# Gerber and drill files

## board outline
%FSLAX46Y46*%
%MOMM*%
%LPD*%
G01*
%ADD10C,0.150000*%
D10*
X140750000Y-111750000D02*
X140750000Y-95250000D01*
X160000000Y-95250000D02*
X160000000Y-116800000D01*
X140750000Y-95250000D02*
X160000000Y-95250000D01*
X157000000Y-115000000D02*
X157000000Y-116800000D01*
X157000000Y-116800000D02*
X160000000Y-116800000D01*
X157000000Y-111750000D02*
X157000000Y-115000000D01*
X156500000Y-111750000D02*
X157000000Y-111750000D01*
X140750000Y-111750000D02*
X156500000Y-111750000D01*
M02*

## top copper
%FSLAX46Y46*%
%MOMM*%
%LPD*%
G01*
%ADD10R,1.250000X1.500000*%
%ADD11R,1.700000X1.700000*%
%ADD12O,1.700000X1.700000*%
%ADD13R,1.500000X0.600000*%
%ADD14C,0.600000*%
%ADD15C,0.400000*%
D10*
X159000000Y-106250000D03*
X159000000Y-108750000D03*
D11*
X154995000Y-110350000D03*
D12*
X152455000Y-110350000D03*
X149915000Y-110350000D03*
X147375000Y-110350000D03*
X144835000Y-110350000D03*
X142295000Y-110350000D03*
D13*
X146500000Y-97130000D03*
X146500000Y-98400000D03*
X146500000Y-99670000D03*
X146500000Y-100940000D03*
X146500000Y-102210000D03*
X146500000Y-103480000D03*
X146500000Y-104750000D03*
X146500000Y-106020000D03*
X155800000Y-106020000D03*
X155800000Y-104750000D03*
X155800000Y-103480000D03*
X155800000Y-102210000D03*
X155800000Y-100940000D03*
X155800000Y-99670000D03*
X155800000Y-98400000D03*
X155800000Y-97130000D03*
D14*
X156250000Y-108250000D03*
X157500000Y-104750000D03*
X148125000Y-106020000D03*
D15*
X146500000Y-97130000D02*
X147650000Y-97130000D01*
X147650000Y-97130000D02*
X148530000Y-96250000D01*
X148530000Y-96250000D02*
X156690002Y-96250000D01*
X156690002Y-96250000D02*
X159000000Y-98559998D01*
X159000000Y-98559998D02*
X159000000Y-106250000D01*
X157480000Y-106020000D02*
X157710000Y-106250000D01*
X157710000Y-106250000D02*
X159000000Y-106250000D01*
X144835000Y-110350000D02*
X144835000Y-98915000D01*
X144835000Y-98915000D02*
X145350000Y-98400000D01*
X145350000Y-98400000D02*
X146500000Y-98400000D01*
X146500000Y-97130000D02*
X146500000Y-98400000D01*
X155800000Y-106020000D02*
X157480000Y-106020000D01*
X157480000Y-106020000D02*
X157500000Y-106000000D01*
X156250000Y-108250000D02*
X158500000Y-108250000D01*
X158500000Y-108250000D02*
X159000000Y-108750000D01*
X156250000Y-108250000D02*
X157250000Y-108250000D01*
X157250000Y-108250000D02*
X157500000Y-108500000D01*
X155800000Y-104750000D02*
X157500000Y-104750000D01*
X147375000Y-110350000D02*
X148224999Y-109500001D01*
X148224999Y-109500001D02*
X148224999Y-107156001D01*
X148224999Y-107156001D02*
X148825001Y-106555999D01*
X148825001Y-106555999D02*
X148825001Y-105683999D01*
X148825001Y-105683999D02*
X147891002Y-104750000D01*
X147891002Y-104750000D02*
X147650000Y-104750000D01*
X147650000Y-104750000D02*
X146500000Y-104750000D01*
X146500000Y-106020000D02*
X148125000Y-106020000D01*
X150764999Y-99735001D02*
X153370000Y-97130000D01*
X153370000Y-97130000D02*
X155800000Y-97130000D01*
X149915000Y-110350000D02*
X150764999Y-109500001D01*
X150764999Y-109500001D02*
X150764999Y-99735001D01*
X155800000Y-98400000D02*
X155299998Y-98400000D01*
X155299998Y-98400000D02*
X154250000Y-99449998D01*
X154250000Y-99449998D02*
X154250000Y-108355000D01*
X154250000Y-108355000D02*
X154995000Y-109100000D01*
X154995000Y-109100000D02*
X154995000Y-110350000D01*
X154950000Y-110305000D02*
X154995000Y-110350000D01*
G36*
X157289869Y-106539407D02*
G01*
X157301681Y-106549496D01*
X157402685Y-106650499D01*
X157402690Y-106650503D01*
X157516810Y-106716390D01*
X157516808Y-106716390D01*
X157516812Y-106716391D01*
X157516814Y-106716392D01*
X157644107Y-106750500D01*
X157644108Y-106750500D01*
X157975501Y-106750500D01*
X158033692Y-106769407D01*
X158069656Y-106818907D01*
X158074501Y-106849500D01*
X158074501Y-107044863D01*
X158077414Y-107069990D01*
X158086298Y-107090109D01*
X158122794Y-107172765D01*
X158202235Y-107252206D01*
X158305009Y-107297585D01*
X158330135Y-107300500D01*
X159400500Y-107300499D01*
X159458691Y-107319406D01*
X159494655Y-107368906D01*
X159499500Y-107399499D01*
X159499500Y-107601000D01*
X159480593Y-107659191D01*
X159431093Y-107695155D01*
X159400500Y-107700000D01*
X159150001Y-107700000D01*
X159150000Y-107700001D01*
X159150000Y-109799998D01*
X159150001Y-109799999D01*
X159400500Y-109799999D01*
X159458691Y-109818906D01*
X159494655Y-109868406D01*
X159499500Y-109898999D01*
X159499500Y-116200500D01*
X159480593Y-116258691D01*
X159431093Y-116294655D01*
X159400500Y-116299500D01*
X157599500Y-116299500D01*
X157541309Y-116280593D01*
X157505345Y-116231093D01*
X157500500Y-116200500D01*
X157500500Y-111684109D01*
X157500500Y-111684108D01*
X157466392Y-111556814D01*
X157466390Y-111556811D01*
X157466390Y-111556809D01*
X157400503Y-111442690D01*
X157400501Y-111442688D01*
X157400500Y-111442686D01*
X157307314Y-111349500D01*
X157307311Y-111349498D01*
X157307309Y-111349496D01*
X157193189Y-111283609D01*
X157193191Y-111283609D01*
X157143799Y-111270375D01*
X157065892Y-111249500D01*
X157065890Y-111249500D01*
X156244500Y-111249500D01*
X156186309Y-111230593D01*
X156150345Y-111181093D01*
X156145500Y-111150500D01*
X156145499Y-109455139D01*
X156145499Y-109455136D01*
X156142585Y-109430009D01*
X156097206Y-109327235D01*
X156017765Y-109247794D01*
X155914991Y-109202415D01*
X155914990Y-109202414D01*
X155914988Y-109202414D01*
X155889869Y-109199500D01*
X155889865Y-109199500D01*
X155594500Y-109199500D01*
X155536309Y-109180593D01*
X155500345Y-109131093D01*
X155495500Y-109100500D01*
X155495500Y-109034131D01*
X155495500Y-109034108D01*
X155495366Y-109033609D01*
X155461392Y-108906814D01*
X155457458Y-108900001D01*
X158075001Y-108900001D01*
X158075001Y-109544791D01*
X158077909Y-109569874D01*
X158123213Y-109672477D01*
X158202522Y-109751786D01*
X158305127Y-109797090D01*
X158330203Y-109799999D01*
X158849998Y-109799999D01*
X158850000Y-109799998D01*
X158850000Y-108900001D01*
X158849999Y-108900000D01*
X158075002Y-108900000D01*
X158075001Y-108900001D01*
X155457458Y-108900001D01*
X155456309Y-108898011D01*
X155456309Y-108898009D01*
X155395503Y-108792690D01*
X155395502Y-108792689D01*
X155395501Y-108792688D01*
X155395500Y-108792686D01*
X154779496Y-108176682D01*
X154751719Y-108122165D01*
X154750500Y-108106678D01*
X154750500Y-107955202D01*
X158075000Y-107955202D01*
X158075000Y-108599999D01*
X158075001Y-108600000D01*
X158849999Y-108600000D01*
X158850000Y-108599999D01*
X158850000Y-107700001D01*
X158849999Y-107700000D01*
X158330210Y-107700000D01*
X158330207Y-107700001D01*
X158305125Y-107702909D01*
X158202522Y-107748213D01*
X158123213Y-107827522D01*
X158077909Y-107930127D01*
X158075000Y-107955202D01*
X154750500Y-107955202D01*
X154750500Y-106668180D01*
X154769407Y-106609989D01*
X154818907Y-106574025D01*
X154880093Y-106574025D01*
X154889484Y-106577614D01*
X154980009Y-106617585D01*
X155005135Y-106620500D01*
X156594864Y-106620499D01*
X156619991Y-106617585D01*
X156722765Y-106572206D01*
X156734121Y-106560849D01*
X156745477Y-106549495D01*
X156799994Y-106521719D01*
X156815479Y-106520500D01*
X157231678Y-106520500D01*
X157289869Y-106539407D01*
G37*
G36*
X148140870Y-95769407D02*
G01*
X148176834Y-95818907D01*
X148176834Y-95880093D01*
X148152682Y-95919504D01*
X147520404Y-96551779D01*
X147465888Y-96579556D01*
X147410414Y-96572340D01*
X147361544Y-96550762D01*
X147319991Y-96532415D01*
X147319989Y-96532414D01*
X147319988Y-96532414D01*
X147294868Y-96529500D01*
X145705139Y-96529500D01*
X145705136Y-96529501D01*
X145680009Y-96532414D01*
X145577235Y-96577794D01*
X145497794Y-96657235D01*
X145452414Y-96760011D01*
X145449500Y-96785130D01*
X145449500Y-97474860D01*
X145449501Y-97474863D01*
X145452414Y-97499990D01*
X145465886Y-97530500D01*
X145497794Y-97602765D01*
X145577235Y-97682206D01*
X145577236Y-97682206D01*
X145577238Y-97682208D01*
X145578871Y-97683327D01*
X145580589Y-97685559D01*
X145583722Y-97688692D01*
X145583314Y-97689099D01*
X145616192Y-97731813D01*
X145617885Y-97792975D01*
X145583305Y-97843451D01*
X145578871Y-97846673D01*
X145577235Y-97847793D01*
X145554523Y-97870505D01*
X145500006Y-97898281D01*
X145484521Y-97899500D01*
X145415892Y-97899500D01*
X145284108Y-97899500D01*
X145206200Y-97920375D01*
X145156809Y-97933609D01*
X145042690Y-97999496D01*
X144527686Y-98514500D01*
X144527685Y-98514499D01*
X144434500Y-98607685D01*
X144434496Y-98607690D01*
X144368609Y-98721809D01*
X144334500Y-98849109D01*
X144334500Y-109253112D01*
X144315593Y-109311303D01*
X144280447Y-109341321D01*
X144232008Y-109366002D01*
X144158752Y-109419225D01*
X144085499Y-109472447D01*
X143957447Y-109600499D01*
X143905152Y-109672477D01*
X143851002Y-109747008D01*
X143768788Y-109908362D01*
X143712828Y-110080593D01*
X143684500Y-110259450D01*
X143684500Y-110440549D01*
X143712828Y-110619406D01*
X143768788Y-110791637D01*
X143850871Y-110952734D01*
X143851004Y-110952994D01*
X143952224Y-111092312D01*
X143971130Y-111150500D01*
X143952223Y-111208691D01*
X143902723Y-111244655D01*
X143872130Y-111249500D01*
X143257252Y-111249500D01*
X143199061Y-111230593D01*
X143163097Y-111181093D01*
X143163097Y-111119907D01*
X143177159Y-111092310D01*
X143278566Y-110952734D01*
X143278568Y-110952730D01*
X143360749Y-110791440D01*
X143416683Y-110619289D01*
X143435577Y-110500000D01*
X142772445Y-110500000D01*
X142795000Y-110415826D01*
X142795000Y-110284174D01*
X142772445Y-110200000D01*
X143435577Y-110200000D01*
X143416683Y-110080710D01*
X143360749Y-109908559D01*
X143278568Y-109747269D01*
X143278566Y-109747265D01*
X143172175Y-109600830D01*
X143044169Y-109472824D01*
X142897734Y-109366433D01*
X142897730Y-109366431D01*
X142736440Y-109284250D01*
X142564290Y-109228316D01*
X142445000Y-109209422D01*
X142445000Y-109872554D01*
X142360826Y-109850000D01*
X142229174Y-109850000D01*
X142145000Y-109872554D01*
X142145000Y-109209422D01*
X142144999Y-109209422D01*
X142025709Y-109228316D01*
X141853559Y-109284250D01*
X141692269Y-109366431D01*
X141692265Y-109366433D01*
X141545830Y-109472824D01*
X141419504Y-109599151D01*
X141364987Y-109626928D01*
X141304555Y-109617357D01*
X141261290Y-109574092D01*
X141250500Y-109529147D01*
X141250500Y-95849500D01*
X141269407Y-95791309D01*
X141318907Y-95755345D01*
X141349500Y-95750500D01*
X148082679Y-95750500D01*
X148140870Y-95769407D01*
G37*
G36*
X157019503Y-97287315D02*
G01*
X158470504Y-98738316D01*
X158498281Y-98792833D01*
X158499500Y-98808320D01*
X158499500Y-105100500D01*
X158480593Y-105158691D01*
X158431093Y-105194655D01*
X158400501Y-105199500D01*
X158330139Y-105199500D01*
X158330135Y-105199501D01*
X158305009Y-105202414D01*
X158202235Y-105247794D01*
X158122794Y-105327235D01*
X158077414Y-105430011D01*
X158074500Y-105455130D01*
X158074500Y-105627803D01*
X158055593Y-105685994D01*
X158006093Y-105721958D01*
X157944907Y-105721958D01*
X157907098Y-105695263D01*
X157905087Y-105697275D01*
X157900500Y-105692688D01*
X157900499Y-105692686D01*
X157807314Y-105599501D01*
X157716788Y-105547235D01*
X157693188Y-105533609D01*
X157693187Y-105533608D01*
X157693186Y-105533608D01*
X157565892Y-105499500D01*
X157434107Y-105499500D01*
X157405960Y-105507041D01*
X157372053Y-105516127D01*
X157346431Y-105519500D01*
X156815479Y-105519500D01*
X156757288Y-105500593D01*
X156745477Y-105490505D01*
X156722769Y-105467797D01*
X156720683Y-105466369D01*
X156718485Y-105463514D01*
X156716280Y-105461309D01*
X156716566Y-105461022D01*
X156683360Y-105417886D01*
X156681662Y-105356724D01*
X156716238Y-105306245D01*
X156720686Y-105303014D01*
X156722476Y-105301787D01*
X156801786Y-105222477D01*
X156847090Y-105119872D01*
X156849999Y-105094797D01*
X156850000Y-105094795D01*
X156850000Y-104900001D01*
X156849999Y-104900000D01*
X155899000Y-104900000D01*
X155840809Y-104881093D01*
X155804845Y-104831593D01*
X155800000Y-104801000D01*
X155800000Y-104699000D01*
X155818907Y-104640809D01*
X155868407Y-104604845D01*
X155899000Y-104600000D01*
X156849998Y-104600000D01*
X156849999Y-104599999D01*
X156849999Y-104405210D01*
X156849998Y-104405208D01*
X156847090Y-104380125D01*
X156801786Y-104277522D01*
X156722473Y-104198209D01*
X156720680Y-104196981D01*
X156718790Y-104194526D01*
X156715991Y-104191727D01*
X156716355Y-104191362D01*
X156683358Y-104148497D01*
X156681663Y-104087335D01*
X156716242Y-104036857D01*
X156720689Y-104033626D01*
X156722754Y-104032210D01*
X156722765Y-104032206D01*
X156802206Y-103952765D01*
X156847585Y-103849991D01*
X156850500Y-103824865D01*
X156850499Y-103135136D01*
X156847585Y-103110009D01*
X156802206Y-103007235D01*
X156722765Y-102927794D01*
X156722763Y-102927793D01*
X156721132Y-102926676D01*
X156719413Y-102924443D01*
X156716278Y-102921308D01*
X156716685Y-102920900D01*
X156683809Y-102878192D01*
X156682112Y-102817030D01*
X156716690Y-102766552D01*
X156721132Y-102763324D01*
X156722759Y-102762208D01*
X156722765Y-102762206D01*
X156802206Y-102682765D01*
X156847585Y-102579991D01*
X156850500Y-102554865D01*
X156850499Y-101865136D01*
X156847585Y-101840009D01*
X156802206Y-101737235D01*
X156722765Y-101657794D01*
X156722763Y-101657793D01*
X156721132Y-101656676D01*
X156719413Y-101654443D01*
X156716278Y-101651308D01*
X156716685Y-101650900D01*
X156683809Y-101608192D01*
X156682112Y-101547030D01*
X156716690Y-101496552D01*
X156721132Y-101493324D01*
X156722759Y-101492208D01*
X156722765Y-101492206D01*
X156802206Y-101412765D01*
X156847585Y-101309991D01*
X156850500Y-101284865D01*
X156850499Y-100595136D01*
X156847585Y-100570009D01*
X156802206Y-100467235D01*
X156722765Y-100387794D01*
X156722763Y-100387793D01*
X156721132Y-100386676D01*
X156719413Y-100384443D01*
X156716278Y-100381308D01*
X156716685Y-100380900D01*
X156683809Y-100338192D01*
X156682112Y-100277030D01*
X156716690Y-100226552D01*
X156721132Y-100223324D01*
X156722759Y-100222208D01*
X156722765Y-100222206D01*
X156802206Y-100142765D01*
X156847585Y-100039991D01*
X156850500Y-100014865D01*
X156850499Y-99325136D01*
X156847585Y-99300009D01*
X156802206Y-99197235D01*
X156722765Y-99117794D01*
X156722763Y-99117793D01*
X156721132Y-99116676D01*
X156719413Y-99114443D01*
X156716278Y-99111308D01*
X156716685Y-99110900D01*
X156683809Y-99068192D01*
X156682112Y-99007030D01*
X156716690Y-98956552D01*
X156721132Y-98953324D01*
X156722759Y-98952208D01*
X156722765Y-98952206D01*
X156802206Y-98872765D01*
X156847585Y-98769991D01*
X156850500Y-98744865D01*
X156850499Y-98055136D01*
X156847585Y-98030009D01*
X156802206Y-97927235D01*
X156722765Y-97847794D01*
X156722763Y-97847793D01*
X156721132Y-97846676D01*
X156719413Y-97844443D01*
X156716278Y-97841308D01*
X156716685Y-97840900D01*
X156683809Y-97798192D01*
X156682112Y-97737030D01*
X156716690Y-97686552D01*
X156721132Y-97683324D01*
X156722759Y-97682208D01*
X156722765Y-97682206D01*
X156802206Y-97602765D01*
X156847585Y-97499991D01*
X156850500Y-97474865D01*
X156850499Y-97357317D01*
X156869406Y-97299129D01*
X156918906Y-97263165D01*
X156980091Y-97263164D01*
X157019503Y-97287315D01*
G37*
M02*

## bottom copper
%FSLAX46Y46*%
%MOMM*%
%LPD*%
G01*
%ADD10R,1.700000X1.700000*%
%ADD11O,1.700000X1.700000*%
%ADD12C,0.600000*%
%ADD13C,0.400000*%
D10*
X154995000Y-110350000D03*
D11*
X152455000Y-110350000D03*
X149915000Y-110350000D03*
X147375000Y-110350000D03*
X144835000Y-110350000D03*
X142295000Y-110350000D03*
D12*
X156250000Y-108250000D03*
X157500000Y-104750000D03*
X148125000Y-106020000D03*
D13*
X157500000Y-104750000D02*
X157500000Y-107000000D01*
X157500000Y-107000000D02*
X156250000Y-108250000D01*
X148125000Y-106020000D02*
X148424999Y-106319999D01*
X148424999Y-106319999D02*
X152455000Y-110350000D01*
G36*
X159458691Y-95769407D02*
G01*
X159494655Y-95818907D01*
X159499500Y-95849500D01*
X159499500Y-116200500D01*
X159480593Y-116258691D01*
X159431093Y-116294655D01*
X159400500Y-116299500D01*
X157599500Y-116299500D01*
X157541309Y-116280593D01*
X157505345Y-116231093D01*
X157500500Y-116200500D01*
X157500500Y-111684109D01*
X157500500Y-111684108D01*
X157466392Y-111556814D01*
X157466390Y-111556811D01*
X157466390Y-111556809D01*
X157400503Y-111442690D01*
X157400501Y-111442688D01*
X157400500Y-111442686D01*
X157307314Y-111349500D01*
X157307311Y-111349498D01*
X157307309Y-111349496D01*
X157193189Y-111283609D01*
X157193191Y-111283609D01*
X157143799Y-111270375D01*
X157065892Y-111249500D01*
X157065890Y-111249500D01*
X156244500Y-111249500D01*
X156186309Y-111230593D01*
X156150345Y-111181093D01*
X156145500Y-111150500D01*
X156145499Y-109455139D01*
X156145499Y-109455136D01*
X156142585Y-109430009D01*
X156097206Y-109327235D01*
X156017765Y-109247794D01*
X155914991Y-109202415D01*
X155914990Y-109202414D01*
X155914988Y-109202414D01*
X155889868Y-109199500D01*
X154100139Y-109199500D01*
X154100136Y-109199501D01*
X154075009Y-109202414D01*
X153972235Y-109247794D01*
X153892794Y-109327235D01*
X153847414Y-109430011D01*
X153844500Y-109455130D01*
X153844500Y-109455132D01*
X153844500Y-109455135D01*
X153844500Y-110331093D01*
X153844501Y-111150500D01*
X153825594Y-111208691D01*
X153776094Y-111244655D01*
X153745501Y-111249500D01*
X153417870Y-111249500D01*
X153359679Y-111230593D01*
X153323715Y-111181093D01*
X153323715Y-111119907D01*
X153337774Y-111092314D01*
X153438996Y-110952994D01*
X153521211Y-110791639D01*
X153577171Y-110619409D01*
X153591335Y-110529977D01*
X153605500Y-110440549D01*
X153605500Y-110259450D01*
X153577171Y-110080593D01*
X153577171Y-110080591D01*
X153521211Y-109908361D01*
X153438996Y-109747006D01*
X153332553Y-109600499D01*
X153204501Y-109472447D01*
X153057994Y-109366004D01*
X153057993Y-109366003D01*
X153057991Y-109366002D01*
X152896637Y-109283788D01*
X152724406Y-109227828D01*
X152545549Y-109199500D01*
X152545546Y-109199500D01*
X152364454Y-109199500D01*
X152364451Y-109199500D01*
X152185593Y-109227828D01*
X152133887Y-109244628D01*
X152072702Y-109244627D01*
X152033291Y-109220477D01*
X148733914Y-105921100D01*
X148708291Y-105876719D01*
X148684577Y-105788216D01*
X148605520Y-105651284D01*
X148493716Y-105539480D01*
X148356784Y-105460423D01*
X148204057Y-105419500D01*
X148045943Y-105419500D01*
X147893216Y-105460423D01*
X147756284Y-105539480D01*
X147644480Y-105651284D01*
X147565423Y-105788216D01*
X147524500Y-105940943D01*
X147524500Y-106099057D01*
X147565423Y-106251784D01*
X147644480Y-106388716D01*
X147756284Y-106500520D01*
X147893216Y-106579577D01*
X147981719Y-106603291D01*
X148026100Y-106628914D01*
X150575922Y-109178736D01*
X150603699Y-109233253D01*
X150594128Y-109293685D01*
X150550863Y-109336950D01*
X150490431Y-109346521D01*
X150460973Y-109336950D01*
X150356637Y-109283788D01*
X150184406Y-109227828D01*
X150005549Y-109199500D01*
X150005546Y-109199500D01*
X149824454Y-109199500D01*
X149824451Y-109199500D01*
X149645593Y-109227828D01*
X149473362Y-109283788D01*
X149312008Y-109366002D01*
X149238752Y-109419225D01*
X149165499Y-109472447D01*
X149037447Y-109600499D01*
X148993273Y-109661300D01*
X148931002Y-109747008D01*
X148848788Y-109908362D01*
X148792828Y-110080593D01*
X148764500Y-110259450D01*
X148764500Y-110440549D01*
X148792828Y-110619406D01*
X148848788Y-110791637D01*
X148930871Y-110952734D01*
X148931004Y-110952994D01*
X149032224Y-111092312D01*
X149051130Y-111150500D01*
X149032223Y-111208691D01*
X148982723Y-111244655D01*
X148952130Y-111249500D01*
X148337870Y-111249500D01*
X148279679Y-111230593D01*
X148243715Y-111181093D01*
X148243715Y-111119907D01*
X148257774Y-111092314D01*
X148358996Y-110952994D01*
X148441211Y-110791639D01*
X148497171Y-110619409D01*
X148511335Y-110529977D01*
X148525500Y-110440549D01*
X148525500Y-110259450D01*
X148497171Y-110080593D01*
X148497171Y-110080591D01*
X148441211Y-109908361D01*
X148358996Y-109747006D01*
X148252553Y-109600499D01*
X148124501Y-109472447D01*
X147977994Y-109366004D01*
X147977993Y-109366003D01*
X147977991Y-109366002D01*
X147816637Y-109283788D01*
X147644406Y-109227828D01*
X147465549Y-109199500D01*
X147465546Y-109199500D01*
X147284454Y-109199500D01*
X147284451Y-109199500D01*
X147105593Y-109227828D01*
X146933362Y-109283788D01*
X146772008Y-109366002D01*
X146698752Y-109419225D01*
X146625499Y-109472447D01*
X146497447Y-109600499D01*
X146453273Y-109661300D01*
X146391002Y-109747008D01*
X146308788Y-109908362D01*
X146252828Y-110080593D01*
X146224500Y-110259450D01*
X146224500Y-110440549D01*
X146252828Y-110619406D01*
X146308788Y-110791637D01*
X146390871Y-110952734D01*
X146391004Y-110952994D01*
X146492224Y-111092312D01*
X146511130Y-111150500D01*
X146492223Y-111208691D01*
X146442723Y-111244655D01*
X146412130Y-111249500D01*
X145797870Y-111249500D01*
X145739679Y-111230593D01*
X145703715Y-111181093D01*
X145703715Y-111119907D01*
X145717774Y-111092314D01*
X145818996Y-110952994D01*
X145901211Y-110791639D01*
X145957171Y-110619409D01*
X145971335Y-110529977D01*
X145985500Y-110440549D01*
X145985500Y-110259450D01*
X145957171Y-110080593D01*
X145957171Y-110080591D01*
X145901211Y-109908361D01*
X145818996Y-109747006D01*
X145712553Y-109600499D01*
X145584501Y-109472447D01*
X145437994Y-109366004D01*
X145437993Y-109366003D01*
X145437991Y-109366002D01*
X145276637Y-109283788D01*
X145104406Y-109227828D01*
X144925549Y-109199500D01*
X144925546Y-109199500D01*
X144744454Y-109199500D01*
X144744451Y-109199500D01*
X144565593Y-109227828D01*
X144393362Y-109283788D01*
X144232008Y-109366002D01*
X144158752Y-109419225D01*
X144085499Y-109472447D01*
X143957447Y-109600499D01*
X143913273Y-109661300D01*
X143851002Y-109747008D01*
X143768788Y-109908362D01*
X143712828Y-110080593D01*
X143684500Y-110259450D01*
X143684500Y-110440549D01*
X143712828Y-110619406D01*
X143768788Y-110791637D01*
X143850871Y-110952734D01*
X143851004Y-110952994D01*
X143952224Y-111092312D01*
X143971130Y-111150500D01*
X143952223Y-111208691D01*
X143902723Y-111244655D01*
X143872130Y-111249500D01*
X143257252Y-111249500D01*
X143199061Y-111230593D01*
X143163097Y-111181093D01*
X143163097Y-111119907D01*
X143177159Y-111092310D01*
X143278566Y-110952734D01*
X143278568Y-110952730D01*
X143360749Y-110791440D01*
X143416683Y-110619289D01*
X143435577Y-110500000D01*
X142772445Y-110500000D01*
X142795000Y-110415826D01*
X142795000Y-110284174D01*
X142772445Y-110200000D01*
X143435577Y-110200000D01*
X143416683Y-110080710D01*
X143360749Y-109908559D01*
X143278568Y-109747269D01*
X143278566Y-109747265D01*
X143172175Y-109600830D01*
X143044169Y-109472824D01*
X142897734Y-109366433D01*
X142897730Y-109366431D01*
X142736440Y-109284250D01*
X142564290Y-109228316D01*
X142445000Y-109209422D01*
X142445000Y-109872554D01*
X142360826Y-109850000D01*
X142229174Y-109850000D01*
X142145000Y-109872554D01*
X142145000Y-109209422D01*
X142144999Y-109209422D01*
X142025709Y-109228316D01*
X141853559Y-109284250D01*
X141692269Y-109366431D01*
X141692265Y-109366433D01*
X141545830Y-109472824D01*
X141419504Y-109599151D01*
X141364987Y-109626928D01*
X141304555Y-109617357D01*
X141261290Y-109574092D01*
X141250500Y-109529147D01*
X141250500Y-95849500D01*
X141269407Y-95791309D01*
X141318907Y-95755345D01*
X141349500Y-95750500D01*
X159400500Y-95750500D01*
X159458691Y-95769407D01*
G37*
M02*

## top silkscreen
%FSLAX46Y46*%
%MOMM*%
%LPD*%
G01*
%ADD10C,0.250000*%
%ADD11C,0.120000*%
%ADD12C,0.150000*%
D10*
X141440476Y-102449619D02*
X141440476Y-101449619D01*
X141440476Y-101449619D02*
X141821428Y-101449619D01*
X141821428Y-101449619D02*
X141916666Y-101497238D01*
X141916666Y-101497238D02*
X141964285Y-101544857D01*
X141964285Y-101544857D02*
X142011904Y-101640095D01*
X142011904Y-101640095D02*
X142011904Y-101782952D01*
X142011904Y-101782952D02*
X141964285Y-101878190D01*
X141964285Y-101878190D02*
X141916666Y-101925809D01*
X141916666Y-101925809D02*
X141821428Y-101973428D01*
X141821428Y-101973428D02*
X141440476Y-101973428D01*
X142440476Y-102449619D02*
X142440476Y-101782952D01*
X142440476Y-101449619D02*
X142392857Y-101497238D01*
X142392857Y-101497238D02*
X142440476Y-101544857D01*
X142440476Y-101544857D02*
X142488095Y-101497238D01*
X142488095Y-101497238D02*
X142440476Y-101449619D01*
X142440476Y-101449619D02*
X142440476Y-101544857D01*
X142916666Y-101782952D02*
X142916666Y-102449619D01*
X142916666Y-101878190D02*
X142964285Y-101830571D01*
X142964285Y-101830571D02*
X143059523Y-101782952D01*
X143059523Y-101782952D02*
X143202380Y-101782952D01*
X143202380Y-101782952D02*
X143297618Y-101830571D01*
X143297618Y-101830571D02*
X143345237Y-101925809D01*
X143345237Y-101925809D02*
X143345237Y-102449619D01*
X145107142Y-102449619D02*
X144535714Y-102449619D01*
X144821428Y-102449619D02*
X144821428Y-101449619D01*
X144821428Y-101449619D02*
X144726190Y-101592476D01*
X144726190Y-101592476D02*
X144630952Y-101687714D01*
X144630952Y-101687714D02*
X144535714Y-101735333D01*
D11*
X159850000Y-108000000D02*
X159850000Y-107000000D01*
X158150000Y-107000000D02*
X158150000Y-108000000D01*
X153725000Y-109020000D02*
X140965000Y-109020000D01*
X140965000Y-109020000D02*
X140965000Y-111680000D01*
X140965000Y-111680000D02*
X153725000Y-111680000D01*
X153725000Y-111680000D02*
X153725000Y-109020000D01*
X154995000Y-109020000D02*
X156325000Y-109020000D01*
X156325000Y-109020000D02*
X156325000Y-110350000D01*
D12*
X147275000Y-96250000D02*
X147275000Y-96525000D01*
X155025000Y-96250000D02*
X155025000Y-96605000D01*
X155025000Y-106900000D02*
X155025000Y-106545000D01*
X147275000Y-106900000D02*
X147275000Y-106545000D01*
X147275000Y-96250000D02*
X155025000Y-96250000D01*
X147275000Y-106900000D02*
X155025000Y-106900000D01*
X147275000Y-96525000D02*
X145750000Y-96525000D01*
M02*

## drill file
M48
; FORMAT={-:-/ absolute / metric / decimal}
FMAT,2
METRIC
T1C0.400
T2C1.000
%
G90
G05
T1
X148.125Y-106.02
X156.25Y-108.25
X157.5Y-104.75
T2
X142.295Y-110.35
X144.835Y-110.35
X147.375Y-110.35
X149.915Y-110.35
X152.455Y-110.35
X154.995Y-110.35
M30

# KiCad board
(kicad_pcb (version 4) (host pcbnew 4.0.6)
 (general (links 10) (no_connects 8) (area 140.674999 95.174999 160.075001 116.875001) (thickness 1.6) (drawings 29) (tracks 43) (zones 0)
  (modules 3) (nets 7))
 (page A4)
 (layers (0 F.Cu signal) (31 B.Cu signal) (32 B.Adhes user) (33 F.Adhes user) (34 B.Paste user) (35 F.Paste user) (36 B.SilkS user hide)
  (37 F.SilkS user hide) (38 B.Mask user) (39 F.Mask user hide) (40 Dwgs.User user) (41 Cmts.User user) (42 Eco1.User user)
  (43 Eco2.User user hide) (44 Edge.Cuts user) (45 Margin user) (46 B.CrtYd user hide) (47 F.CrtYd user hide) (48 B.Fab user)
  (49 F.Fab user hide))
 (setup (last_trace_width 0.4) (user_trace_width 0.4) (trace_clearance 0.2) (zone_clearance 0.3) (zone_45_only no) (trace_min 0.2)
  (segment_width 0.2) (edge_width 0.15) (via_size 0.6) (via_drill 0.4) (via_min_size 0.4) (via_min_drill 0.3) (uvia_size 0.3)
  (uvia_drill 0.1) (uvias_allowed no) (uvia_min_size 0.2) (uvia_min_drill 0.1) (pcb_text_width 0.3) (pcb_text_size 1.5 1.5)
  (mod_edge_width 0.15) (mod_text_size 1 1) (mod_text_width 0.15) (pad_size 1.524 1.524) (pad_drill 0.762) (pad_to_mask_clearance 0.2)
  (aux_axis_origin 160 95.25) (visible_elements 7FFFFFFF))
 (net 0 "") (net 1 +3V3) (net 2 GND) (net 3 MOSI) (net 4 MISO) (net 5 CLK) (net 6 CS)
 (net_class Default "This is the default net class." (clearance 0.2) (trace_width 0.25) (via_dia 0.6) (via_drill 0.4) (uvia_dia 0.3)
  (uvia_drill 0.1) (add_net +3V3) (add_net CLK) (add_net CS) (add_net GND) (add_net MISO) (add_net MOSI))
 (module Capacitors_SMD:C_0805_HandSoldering (layer F.Cu) (at 159 107.5 270)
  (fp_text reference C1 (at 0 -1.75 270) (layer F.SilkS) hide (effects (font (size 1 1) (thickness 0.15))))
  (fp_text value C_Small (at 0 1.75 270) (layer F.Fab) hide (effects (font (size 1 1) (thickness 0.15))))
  (fp_line (start 0.5 -0.85) (end -0.5 -0.85) (layer F.SilkS) (width 0.12))
  (fp_line (start -0.5 0.85) (end 0.5 0.85) (layer F.SilkS) (width 0.12))
  (pad 1 smd rect (at -1.25 0 270) (size 1.5 1.25) (layers F.Cu F.Paste F.Mask) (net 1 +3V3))
  (pad 2 smd rect (at 1.25 0 270) (size 1.5 1.25) (layers F.Cu F.Paste F.Mask) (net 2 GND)))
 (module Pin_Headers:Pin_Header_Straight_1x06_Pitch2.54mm (layer F.Cu) (at 154.995 110.35 270)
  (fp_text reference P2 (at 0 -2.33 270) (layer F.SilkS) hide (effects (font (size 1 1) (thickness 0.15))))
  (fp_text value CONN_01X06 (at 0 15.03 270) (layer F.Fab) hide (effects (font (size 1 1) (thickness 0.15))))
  (fp_line (start -1.33 1.27) (end -1.33 14.03) (layer F.SilkS) (width 0.12))
  (fp_line (start -1.33 14.03) (end 1.33 14.03) (layer F.SilkS) (width 0.12))
  (fp_line (start 1.33 14.03) (end 1.33 1.27) (layer F.SilkS) (width 0.12))
  (fp_line (start 1.33 1.27) (end -1.33 1.27) (layer F.SilkS) (width 0.12))
  (fp_line (start -1.33 0) (end -1.33 -1.33) (layer F.SilkS) (width 0.12))
  (fp_line (start -1.33 -1.33) (end 0 -1.33) (layer F.SilkS) (width 0.12))
  (pad 1 thru_hole rect (at 0 0 270) (size 1.7 1.7) (drill 1) (layers *.Cu *.Mask) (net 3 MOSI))
  (pad 2 thru_hole oval (at 0 2.54 270) (size 1.7 1.7) (drill 1) (layers *.Cu *.Mask) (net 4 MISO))
  (pad 3 thru_hole oval (at 0 5.08 270) (size 1.7 1.7) (drill 1) (layers *.Cu *.Mask) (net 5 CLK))
  (pad 4 thru_hole oval (at 0 7.62 270) (size 1.7 1.7) (drill 1) (layers *.Cu *.Mask) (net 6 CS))
  (pad 5 thru_hole oval (at 0 10.16 270) (size 1.7 1.7) (drill 1) (layers *.Cu *.Mask) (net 1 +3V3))
  (pad 6 thru_hole oval (at 0 12.7 270) (size 1.7 1.7) (drill 1) (layers *.Cu *.Mask) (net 2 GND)))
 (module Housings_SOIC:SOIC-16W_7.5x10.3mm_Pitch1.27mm (layer F.Cu) (at 151.15 101.575)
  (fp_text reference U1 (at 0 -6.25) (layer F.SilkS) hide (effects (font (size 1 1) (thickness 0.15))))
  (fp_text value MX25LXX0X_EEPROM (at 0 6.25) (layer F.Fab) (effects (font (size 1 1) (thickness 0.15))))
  (fp_line (start -3.875 -5.325) (end -3.875 -5.05) (layer F.SilkS) (width 0.15))
  (fp_line (start 3.875 -5.325) (end 3.875 -4.97) (layer F.SilkS) (width 0.15))
  (fp_line (start 3.875 5.325) (end 3.875 4.97) (layer F.SilkS) (width 0.15))
  (fp_line (start -3.875 5.325) (end -3.875 4.97) (layer F.SilkS) (width 0.15))
  (fp_line (start -3.875 -5.325) (end 3.875 -5.325) (layer F.SilkS) (width 0.15))
  (fp_line (start -3.875 5.325) (end 3.875 5.325) (layer F.SilkS) (width 0.15))
  (fp_line (start -3.875 -5.05) (end -5.4 -5.05) (layer F.SilkS) (width 0.15))
  (pad 1 smd rect (at -4.65 -4.445) (size 1.5 0.6) (layers F.Cu F.Paste F.Mask) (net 1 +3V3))
  (pad 2 smd rect (at -4.65 -3.175) (size 1.5 0.6) (layers F.Cu F.Paste F.Mask) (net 1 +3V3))
  (pad 3 smd rect (at -4.65 -1.905) (size 1.5 0.6) (layers F.Cu F.Paste F.Mask))
  (pad 4 smd rect (at -4.65 -0.635) (size 1.5 0.6) (layers F.Cu F.Paste F.Mask))
  (pad 5 smd rect (at -4.65 0.635) (size 1.5 0.6) (layers F.Cu F.Paste F.Mask))
  (pad 6 smd rect (at -4.65 1.905) (size 1.5 0.6) (layers F.Cu F.Paste F.Mask))
  (pad 7 smd rect (at -4.65 3.175) (size 1.5 0.6) (layers F.Cu F.Paste F.Mask) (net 6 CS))
  (pad 8 smd rect (at -4.65 4.445) (size 1.5 0.6) (layers F.Cu F.Paste F.Mask) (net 4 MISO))
  (pad 9 smd rect (at 4.65 4.445) (size 1.5 0.6) (layers F.Cu F.Paste F.Mask) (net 1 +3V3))
  (pad 10 smd rect (at 4.65 3.175) (size 1.5 0.6) (layers F.Cu F.Paste F.Mask) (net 2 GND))
  (pad 11 smd rect (at 4.65 1.905) (size 1.5 0.6) (layers F.Cu F.Paste F.Mask))
  (pad 12 smd rect (at 4.65 0.635) (size 1.5 0.6) (layers F.Cu F.Paste F.Mask))
  (pad 13 smd rect (at 4.65 -0.635) (size 1.5 0.6) (layers F.Cu F.Paste F.Mask))
  (pad 14 smd rect (at 4.65 -1.905) (size 1.5 0.6) (layers F.Cu F.Paste F.Mask))
  (pad 15 smd rect (at 4.65 -3.175) (size 1.5 0.6) (layers F.Cu F.Paste F.Mask) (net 3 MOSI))
  (pad 16 smd rect (at 4.65 -4.445) (size 1.5 0.6) (layers F.Cu F.Paste F.Mask) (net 5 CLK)))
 (gr_line (start 140.75 111.75) (end 140.75 95.25) (layer Edge.Cuts) (width 0.15))
 (gr_line (start 160 95.25) (end 160 116.8) (layer Edge.Cuts) (width 0.15))
 (gr_line (start 140.75 95.25) (end 160 95.25) (layer Edge.Cuts) (width 0.15))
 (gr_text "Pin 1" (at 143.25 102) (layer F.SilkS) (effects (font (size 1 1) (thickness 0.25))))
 (gr_line (start 157 115) (end 157 116.8) (layer Edge.Cuts) (width 0.15))
 (gr_line (start 157 116.8) (end 160 116.8) (layer Edge.Cuts) (width 0.15))
 (gr_line (start 157 111.75) (end 157 115) (layer Edge.Cuts) (width 0.15))
 (gr_line (start 156.5 111.75) (end 157 111.75) (layer Edge.Cuts) (width 0.15))
 (gr_line (start 140.75 111.75) (end 156.5 111.75) (layer Edge.Cuts) (width 0.15))
 (segment (start 146.5 97.13) (end 147.65 97.13) (width 0.4) (layer F.Cu) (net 1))
 (segment (start 147.65 97.13) (end 148.53 96.25) (width 0.4) (layer F.Cu) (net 1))
 (segment (start 148.53 96.25) (end 156.690002 96.25) (width 0.4) (layer F.Cu) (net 1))
 (segment (start 156.690002 96.25) (end 159 98.559998) (width 0.4) (layer F.Cu) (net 1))
 (segment (start 159 98.559998) (end 159 106.25) (width 0.4) (layer F.Cu) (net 1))
 (segment (start 157.48 106.02) (end 157.71 106.25) (width 0.4) (layer F.Cu) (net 1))
 (segment (start 157.71 106.25) (end 159 106.25) (width 0.4) (layer F.Cu) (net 1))
 (segment (start 144.835 110.35) (end 144.835 98.915) (width 0.4) (layer F.Cu) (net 1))
 (segment (start 144.835 98.915) (end 145.35 98.4) (width 0.4) (layer F.Cu) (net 1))
 (segment (start 145.35 98.4) (end 146.5 98.4) (width 0.4) (layer F.Cu) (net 1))
 (segment (start 146.5 97.13) (end 146.5 98.4) (width 0.4) (layer F.Cu) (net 1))
 (segment (start 155.8 106.02) (end 157.48 106.02) (width 0.4) (layer F.Cu) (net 1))
 (segment (start 157.48 106.02) (end 157.5 106) (width 0.4) (layer F.Cu) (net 1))
 (segment (start 156.25 108.25) (end 158.5 108.25) (width 0.4) (layer F.Cu) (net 2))
 (segment (start 158.5 108.25) (end 159 108.75) (width 0.4) (layer F.Cu) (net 2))
 (segment (start 156.25 108.25) (end 157.25 108.25) (width 0.4) (layer F.Cu) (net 2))
 (segment (start 157.25 108.25) (end 157.5 108.5) (width 0.4) (layer F.Cu) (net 2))
 (segment (start 157.5 104.75) (end 157.5 107) (width 0.4) (layer B.Cu) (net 2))
 (segment (start 157.5 107) (end 156.25 108.25) (width 0.4) (layer B.Cu) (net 2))
 (via (at 156.25 108.25) (size 0.6) (drill 0.4) (layers F.Cu B.Cu) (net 2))
 (segment (start 155.8 104.75) (end 157.5 104.75) (width 0.4) (layer F.Cu) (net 2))
 (via (at 157.5 104.75) (size 0.6) (drill 0.4) (layers F.Cu B.Cu) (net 2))
 (segment (start 147.375 110.35) (end 148.224999 109.500001) (width 0.4) (layer F.Cu) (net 6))
 (segment (start 148.224999 109.500001) (end 148.224999 107.156001) (width 0.4) (layer F.Cu) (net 6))
 (segment (start 148.224999 107.156001) (end 148.825001 106.555999) (width 0.4) (layer F.Cu) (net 6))
 (segment (start 148.825001 106.555999) (end 148.825001 105.683999) (width 0.4) (layer F.Cu) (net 6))
 (segment (start 148.825001 105.683999) (end 147.891002 104.75) (width 0.4) (layer F.Cu) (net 6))
 (segment (start 147.891002 104.75) (end 147.65 104.75) (width 0.4) (layer F.Cu) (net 6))
 (segment (start 147.65 104.75) (end 146.5 104.75) (width 0.4) (layer F.Cu) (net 6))
 (segment (start 148.125 106.02) (end 148.424999 106.319999) (width 0.4) (layer B.Cu) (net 4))
 (segment (start 148.424999 106.319999) (end 152.455 110.35) (width 0.4) (layer B.Cu) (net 4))
 (via (at 148.125 106.02) (size 0.6) (drill 0.4) (layers F.Cu B.Cu) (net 4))
 (segment (start 146.5 106.02) (end 148.125 106.02) (width 0.4) (layer F.Cu) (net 4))
 (segment (start 150.764999 99.735001) (end 153.37 97.13) (width 0.4) (layer F.Cu) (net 5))
 (segment (start 153.37 97.13) (end 155.8 97.13) (width 0.4) (layer F.Cu) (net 5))
 (segment (start 149.915 110.35) (end 150.764999 109.500001) (width 0.4) (layer F.Cu) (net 5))
 (segment (start 150.764999 109.500001) (end 150.764999 99.735001) (width 0.4) (layer F.Cu) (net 5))
 (segment (start 155.8 98.4) (end 155.299998 98.4) (width 0.4) (layer F.Cu) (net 3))
 (segment (start 155.299998 98.4) (end 154.25 99.449998) (width 0.4) (layer F.Cu) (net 3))
 (segment (start 154.25 99.449998) (end 154.25 108.355) (width 0.4) (layer F.Cu) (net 3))
 (segment (start 154.25 108.355) (end 154.995 109.1) (width 0.4) (layer F.Cu) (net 3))
 (segment (start 154.995 109.1) (end 154.995 110.35) (width 0.4) (layer F.Cu) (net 3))
 (segment (start 154.95 110.305) (end 154.995 110.35) (width 0.4) (layer F.Cu) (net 3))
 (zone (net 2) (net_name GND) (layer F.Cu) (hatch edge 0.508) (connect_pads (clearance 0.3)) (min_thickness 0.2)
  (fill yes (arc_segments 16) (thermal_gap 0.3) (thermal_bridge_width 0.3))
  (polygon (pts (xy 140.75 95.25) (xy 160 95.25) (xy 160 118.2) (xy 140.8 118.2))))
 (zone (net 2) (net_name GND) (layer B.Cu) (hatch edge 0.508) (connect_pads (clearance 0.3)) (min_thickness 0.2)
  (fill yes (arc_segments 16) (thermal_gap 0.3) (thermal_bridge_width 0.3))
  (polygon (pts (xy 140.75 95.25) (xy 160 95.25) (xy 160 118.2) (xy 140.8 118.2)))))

